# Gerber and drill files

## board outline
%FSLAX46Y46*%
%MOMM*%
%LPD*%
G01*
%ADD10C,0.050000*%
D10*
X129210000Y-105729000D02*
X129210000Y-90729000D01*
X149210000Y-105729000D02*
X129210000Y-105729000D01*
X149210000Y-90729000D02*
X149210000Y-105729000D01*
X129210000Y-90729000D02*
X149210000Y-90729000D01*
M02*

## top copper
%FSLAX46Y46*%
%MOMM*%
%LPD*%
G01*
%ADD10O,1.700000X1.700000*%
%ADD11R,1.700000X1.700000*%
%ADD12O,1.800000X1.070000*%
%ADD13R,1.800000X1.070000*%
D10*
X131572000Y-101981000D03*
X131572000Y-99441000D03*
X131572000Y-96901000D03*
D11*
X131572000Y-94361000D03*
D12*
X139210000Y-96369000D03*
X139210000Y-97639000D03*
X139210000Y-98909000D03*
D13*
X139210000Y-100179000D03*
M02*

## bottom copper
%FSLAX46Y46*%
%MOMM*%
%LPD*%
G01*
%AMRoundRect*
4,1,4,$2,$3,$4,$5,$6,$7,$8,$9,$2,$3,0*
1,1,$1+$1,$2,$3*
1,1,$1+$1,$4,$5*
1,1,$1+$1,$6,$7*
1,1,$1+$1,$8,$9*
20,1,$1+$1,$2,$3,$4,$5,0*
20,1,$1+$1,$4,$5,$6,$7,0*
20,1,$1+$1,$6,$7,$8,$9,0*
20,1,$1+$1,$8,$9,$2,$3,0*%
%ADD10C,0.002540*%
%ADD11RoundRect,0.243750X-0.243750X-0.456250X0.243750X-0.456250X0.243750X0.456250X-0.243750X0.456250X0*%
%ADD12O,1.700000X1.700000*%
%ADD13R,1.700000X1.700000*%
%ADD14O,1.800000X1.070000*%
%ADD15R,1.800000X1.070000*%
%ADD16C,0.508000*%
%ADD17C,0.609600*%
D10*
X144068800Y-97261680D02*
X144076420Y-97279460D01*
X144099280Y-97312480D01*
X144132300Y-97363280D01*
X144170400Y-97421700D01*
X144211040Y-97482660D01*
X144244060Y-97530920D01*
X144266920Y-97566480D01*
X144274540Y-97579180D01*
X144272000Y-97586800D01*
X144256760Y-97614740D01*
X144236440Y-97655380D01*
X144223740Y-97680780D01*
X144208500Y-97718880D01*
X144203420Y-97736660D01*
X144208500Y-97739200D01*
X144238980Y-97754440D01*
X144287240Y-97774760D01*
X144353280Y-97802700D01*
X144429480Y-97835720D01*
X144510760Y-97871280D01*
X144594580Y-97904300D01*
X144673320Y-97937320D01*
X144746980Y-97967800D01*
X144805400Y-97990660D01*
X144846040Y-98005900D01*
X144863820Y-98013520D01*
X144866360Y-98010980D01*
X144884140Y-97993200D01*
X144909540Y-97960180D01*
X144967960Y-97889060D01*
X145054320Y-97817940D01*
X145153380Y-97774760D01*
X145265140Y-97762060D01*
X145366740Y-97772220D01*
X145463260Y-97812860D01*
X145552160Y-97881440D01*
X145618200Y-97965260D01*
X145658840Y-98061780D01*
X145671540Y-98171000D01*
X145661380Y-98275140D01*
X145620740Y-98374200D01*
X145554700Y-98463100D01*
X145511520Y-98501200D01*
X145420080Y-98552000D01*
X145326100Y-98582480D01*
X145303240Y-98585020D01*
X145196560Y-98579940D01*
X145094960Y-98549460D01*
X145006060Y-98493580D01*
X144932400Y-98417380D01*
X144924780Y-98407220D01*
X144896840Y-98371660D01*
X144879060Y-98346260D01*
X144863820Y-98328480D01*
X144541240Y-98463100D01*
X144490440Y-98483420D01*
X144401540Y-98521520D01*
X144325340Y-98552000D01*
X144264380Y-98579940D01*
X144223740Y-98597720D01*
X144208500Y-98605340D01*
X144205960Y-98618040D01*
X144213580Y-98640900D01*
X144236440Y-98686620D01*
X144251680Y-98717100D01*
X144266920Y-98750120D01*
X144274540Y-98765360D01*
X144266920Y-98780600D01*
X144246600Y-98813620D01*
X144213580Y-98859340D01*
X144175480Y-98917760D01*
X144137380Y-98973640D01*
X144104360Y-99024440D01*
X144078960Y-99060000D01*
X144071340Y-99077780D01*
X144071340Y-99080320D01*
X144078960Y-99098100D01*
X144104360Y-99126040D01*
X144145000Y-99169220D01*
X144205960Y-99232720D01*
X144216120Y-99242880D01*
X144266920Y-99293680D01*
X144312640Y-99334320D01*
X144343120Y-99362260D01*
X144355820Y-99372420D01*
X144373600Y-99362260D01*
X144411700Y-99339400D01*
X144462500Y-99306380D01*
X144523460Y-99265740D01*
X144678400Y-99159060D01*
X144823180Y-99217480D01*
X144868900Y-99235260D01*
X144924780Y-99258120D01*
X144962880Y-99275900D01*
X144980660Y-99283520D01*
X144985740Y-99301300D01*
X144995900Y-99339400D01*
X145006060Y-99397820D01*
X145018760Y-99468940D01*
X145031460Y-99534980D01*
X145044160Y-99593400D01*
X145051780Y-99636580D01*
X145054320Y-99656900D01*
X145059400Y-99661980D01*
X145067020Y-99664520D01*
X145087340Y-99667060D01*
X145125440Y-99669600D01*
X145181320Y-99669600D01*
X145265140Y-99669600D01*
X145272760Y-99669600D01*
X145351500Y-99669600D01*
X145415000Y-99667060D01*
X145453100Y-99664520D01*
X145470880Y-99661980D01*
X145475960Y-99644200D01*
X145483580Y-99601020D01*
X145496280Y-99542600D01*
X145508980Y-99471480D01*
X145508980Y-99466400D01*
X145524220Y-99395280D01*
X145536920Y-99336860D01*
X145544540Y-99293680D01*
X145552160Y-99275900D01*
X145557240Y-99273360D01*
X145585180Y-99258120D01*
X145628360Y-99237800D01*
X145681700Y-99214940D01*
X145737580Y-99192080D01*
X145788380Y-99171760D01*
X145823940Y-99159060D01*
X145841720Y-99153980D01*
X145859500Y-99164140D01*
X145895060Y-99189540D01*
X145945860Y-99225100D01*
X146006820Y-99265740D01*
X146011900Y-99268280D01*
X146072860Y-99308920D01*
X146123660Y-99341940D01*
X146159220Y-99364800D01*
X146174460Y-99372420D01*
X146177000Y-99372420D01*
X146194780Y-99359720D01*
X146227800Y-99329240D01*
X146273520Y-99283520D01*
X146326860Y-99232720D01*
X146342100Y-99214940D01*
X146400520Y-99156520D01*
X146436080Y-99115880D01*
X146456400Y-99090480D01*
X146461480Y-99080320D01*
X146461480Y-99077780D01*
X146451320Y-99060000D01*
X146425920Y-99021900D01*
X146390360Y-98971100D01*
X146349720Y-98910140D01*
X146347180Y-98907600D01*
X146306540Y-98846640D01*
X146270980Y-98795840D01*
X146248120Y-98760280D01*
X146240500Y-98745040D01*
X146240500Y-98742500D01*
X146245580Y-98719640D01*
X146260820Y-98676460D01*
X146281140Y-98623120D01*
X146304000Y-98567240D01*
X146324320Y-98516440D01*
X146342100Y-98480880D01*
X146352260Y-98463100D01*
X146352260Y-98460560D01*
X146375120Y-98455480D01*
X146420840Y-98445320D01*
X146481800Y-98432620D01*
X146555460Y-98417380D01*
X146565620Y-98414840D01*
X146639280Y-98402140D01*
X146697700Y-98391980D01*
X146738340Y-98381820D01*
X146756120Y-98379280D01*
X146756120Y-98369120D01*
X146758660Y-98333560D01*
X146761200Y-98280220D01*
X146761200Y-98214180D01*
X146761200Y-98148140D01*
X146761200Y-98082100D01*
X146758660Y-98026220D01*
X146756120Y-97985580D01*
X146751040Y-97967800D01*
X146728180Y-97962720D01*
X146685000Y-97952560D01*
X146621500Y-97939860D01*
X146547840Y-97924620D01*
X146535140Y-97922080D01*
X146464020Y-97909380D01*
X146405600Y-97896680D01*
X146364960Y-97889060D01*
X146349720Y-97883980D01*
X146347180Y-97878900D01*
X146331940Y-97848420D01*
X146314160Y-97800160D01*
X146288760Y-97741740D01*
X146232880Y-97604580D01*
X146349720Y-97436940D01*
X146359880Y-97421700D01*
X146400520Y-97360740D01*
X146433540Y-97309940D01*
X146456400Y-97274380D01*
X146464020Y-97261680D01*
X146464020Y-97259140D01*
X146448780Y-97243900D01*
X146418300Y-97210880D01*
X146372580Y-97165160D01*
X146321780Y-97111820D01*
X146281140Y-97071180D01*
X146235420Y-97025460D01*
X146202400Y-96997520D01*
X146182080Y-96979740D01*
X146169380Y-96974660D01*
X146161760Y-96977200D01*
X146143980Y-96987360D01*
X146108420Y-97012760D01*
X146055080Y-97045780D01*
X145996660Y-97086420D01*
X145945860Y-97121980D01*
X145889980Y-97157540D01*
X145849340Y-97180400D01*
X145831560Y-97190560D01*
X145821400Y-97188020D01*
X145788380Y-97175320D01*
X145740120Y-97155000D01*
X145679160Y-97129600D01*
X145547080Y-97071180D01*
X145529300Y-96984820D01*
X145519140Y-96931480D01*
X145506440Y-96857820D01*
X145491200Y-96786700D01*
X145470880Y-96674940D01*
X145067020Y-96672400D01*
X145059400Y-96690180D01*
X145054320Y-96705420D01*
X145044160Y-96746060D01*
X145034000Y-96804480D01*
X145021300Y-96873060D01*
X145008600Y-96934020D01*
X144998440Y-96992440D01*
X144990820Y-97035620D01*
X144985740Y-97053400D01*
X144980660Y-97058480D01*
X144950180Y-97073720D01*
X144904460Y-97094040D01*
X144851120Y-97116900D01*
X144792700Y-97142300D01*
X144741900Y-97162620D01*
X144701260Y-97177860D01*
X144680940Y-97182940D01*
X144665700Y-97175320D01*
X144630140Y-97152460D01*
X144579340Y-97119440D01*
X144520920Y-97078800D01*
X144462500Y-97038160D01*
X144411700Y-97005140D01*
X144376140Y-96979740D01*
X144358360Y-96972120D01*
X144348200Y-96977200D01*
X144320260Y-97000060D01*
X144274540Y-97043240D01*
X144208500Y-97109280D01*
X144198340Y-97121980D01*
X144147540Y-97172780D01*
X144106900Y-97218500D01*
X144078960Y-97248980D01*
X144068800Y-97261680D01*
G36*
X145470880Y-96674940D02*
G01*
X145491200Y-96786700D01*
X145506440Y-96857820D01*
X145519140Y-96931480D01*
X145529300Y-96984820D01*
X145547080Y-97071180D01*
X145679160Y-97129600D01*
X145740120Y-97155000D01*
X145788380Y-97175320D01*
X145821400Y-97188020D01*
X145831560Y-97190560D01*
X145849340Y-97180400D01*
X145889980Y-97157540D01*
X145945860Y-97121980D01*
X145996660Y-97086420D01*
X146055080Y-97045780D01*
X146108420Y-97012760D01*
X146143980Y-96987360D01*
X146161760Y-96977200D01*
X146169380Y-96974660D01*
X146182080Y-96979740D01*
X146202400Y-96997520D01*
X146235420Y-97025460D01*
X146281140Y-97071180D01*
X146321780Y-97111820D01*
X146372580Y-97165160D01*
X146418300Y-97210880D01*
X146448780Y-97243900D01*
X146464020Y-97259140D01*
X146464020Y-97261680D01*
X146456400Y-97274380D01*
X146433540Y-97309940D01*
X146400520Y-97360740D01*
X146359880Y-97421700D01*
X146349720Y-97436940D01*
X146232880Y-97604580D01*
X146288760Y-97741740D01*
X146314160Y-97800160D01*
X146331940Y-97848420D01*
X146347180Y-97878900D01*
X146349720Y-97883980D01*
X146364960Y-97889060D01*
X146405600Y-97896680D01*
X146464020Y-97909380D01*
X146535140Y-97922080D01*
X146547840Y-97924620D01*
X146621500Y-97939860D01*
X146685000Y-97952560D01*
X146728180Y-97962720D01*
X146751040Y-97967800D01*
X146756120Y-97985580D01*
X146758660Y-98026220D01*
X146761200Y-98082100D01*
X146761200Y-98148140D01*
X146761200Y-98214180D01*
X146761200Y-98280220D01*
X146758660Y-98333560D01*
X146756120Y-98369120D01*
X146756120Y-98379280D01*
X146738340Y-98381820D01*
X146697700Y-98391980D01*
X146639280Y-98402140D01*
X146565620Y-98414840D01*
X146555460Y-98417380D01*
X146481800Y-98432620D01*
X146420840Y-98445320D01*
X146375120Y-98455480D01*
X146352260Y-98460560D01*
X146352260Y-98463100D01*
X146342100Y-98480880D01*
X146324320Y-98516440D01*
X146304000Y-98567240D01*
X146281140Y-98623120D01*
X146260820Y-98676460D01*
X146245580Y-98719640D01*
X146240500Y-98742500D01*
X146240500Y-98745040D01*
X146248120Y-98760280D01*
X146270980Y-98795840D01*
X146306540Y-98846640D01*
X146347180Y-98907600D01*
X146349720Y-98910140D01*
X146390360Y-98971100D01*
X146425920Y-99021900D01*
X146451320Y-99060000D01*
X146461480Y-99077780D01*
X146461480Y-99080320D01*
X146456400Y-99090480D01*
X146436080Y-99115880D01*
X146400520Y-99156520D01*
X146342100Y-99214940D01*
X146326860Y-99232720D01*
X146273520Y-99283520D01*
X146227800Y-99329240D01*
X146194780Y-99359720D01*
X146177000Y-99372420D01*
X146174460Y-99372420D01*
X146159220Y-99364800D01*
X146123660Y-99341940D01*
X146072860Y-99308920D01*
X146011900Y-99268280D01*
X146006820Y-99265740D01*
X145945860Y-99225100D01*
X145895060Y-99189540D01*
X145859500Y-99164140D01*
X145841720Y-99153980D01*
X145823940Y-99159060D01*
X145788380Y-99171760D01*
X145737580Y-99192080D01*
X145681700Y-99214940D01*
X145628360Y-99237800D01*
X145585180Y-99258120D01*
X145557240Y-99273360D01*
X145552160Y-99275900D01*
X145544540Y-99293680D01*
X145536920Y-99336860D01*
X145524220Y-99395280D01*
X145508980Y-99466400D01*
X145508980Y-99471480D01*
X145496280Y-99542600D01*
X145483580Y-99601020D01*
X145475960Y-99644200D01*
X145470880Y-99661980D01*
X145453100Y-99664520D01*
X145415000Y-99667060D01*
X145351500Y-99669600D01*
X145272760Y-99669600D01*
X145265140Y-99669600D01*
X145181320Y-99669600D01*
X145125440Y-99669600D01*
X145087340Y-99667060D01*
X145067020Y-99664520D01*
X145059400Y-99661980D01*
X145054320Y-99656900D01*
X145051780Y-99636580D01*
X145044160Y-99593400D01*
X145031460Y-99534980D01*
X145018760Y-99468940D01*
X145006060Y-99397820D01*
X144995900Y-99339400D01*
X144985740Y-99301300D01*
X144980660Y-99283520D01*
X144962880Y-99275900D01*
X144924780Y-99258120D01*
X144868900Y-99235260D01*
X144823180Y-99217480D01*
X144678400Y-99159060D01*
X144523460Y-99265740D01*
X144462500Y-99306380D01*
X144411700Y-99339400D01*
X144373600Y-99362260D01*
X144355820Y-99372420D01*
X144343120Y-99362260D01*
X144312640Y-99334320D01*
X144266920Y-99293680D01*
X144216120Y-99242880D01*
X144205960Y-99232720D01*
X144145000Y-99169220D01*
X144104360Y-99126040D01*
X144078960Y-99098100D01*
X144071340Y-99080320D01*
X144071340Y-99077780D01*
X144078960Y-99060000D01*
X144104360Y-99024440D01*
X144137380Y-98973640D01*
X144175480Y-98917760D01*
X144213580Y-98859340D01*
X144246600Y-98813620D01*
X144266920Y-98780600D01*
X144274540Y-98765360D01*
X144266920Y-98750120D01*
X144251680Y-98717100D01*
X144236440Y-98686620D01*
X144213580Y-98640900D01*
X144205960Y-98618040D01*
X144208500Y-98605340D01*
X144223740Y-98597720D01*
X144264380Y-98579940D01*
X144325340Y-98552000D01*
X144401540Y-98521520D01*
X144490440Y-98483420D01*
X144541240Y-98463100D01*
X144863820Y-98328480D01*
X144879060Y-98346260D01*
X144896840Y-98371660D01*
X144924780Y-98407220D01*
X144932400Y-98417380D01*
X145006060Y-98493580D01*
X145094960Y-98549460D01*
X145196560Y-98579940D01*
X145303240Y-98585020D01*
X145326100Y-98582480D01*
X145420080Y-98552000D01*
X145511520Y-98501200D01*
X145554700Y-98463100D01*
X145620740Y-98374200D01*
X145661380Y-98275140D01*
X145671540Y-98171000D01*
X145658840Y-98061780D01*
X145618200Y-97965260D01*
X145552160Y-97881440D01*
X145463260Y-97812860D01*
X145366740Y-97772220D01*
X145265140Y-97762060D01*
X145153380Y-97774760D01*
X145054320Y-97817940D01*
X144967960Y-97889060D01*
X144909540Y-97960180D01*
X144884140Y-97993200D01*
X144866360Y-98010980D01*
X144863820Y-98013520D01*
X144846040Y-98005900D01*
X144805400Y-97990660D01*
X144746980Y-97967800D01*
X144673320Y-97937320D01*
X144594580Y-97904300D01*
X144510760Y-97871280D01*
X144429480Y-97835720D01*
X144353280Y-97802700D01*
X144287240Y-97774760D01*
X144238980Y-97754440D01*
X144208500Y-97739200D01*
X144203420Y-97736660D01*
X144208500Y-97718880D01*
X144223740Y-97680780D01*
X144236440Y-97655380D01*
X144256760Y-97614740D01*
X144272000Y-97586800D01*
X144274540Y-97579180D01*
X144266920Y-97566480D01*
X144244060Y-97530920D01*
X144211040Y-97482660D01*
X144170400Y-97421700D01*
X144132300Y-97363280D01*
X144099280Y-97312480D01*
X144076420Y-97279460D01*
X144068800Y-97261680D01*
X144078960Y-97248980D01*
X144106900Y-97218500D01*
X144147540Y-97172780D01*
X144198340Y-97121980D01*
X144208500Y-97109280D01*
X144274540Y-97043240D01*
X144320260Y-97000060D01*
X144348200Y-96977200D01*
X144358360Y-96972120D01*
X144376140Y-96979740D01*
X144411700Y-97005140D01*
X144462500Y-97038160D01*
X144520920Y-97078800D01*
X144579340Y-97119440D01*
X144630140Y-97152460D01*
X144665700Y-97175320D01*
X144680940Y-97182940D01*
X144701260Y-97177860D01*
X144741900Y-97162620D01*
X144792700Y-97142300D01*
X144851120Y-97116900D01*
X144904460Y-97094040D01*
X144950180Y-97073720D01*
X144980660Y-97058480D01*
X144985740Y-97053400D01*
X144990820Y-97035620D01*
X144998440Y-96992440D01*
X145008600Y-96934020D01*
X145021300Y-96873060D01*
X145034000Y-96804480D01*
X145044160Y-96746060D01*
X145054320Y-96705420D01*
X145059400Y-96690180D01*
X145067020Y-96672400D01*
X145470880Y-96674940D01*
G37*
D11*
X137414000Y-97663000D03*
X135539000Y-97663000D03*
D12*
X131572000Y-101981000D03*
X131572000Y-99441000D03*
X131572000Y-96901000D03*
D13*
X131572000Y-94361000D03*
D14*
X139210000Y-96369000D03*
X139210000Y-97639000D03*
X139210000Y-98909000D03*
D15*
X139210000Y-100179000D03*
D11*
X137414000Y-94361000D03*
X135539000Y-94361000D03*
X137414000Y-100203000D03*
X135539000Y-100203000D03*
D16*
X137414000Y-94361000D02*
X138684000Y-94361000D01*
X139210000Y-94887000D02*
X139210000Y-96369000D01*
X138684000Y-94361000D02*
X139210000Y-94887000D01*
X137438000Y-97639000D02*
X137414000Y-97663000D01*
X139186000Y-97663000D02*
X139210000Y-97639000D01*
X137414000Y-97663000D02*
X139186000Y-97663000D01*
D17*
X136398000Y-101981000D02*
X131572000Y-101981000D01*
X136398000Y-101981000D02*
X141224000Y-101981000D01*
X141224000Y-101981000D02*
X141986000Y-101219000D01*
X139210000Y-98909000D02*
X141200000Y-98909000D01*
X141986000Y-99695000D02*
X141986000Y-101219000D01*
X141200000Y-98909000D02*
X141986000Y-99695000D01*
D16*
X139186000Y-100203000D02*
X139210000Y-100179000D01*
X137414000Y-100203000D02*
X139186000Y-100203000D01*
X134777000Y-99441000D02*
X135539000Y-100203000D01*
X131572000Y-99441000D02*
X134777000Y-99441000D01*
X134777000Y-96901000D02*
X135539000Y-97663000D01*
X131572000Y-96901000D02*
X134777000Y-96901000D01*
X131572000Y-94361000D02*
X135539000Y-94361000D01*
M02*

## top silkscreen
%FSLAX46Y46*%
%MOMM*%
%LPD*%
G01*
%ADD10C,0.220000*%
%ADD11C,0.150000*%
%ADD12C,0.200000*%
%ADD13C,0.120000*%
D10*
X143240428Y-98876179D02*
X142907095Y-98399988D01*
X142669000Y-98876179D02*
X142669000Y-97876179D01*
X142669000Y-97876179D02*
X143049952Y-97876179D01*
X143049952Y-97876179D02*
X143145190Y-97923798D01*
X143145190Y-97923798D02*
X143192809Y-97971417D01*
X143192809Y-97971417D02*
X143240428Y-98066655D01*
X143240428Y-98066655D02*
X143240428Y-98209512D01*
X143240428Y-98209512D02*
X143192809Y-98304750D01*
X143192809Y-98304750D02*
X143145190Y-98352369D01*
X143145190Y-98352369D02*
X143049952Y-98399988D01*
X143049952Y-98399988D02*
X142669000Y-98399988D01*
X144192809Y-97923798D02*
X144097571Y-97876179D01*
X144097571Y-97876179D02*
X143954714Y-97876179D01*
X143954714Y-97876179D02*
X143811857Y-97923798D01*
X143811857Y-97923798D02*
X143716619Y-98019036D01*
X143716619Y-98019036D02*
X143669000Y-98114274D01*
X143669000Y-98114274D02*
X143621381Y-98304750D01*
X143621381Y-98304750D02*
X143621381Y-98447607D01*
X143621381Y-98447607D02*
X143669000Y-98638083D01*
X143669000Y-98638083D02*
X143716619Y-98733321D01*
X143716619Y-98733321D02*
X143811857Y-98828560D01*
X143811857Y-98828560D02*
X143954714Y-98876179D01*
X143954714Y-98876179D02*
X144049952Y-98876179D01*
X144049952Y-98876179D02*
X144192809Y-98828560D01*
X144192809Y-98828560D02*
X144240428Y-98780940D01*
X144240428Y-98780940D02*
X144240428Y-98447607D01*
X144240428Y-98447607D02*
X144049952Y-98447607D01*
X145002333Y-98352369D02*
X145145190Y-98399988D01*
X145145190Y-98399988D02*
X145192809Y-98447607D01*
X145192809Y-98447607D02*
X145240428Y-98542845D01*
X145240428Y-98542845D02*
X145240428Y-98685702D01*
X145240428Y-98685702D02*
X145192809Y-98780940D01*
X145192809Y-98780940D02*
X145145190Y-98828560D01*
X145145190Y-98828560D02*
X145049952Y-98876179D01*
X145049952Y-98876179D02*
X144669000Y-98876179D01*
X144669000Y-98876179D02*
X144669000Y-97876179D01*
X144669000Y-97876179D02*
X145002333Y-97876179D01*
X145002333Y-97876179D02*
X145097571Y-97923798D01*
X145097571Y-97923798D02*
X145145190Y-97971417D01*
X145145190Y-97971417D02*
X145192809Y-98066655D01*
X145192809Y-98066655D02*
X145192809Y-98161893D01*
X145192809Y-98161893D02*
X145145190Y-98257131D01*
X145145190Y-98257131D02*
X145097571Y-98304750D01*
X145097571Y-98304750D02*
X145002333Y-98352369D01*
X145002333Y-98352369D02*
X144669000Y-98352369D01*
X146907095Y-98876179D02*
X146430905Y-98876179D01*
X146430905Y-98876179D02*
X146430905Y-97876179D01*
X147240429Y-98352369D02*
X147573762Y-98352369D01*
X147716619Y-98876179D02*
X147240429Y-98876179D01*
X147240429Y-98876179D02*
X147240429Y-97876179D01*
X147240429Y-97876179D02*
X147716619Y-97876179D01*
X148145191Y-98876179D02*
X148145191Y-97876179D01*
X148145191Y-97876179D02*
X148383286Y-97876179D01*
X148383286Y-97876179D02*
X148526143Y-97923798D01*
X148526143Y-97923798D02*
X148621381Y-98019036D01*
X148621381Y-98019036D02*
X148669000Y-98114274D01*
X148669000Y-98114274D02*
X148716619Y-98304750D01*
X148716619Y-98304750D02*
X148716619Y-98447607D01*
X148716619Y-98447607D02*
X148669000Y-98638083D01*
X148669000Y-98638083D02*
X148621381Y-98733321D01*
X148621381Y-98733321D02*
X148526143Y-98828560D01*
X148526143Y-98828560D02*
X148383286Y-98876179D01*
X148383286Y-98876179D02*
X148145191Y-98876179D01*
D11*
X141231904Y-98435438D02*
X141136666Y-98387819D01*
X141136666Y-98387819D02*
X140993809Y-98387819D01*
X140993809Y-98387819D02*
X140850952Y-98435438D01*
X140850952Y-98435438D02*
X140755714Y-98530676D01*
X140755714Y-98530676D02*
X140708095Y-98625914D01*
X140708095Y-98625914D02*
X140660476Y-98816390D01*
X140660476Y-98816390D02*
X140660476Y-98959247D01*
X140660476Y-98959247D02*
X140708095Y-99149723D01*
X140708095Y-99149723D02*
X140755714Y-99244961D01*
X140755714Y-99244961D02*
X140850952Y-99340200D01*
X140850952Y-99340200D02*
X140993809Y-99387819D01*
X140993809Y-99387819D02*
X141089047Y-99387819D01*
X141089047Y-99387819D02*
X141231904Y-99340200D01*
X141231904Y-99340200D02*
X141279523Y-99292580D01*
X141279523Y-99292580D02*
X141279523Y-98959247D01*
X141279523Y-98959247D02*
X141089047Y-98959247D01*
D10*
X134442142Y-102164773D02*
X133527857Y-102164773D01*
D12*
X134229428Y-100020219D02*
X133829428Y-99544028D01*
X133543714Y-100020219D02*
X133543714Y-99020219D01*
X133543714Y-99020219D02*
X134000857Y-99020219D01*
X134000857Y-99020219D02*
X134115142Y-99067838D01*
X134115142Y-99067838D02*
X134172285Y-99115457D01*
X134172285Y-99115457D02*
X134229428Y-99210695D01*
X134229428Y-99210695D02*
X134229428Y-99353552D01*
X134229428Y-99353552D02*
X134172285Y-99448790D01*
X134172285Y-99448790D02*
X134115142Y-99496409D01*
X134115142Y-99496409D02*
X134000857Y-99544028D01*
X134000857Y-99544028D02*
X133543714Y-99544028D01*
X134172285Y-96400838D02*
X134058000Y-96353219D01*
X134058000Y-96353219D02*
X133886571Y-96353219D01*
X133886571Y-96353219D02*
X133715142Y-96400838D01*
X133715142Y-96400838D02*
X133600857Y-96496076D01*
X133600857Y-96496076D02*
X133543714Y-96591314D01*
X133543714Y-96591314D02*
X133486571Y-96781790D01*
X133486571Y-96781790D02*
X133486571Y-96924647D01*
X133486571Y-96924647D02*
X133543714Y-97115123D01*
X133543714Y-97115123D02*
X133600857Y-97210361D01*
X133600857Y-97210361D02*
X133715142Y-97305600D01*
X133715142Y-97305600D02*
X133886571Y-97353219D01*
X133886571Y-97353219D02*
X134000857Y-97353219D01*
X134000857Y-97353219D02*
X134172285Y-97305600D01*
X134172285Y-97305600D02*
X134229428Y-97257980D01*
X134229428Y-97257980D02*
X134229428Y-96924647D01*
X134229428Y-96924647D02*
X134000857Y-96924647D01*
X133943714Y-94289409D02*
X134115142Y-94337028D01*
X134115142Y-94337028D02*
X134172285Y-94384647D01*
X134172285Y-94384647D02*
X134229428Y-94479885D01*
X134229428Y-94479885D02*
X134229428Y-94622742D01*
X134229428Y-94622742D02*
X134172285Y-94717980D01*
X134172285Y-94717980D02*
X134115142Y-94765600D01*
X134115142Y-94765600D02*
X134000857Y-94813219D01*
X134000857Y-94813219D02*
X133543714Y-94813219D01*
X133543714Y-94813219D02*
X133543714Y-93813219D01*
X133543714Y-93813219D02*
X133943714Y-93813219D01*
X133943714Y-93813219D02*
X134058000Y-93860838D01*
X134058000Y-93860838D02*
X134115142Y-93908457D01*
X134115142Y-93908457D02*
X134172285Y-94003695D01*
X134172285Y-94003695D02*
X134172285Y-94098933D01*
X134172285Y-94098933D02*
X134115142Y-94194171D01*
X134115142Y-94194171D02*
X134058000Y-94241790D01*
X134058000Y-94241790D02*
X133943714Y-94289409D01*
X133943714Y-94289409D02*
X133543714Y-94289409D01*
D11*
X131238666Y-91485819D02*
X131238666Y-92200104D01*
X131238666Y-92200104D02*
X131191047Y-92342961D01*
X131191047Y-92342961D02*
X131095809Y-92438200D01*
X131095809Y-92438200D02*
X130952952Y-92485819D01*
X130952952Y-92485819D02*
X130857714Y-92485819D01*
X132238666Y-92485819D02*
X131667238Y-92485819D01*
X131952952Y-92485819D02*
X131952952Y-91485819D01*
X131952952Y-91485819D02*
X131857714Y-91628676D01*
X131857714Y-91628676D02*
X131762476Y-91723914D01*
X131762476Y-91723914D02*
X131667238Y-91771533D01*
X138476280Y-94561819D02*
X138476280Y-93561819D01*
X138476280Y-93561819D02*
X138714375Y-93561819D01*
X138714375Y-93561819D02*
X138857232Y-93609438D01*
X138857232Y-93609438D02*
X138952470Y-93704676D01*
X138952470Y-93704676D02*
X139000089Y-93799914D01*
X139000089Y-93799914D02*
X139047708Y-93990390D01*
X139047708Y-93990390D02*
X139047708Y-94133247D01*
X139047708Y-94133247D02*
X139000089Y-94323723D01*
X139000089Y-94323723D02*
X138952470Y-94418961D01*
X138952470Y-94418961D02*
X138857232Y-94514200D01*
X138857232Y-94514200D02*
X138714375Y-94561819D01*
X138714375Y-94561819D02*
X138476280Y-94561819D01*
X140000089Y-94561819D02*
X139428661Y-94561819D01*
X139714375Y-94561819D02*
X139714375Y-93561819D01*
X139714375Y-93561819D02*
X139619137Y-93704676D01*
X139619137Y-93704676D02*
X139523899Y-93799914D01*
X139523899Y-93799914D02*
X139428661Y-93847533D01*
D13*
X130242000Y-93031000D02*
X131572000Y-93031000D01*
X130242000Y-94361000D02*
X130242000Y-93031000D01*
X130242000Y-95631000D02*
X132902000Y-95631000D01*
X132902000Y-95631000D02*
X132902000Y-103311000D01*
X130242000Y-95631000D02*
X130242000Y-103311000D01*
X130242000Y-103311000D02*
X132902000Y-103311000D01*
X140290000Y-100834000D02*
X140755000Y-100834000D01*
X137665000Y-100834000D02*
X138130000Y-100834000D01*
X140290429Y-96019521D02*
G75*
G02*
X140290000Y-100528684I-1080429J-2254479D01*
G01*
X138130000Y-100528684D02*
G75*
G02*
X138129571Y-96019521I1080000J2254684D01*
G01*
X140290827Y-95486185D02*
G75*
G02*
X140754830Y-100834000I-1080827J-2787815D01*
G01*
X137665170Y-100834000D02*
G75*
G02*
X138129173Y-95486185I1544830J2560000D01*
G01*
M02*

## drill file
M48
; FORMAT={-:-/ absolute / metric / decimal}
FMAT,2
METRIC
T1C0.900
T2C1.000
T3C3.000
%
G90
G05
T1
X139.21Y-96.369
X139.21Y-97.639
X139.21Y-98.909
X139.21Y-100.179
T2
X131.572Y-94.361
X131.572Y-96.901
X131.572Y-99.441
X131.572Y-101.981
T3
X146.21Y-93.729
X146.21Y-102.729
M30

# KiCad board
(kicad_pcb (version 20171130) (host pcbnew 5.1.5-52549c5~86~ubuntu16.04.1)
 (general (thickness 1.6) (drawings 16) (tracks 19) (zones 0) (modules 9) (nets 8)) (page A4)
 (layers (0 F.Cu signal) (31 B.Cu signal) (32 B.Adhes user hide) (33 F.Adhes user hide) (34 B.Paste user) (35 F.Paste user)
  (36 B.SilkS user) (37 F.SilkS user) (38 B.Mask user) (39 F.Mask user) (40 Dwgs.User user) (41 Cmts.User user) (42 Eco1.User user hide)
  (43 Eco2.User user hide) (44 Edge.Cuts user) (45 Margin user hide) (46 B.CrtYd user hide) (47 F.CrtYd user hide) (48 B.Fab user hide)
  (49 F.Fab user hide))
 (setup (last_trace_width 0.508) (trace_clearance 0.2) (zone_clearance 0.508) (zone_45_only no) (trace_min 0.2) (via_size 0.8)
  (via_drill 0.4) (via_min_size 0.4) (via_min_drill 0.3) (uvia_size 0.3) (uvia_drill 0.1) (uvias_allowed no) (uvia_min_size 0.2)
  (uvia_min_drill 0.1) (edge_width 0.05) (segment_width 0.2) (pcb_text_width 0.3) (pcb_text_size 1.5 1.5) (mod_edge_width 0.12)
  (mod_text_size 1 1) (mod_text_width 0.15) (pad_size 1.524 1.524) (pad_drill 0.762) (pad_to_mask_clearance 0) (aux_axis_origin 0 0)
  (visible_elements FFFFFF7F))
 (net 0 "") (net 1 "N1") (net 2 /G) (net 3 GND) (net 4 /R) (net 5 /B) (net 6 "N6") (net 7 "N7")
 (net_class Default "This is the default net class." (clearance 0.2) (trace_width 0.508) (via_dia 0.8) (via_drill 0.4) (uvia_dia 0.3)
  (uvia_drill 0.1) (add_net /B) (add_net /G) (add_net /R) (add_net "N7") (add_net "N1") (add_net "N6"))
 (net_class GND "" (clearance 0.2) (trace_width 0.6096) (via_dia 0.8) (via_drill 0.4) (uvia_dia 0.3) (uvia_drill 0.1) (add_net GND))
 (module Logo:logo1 (layer B.Cu) (at 141.986 98.171 90)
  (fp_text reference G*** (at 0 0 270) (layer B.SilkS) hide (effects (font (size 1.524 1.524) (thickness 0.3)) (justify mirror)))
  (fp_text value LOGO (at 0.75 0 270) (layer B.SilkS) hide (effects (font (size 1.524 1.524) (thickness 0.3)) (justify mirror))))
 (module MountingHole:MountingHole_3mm (layer F.Cu) (at 146.21 102.729)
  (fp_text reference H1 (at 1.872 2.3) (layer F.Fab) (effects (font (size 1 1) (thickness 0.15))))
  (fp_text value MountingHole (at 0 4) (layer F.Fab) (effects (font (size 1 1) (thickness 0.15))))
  (pad 1 np_thru_hole circle (at 0 0) (size 3 3) (drill 3) (layers *.Cu *.Mask)))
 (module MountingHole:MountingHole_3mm (layer F.Cu) (at 146.21 93.729)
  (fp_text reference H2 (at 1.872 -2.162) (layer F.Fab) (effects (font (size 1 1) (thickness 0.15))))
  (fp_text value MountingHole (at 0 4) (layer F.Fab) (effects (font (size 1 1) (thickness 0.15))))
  (pad 1 np_thru_hole circle (at 0 0) (size 3 3) (drill 3) (layers *.Cu *.Mask)))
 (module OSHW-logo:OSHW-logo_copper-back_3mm (layer B.Cu) (at 145.415 98.171 90)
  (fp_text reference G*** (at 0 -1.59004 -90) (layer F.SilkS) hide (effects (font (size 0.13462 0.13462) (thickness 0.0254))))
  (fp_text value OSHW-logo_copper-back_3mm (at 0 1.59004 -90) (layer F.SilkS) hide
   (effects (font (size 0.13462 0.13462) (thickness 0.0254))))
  (fp_poly
   (pts (xy 0.90932 -1.3462) (xy 0.89154 -1.33858) (xy 0.85852 -1.31572) (xy 0.80772 -1.2827) (xy 0.7493 -1.2446) (xy 0.68834 -1.20396)
    (xy 0.64008 -1.17094) (xy 0.60452 -1.14808) (xy 0.59182 -1.14046) (xy 0.5842 -1.143) (xy 0.55626 -1.15824) (xy 0.51562 -1.17856)
    (xy 0.49022 -1.19126) (xy 0.45212 -1.2065) (xy 0.43434 -1.21158) (xy 0.4318 -1.2065) (xy 0.41656 -1.17602) (xy 0.39624 -1.12776)
    (xy 0.3683 -1.06172) (xy 0.33528 -0.98552) (xy 0.29972 -0.90424) (xy 0.2667 -0.82042) (xy 0.23368 -0.74168) (xy 0.2032 -0.66802)
    (xy 0.18034 -0.6096) (xy 0.1651 -0.56896) (xy 0.15748 -0.55118) (xy 0.16002 -0.54864) (xy 0.1778 -0.53086) (xy 0.21082 -0.50546)
    (xy 0.28194 -0.44704) (xy 0.35306 -0.36068) (xy 0.39624 -0.26162) (xy 0.40894 -0.14986) (xy 0.39878 -0.04826) (xy 0.35814 0.04826)
    (xy 0.28956 0.13716) (xy 0.20574 0.2032) (xy 0.10922 0.24384) (xy 0 0.25654) (xy -0.10414 0.24638) (xy -0.2032 0.20574)
    (xy -0.2921 0.1397) (xy -0.3302 0.09652) (xy -0.381 0.00508) (xy -0.41148 -0.0889) (xy -0.41402 -0.11176) (xy -0.40894 -0.21844)
    (xy -0.37846 -0.32004) (xy -0.32258 -0.40894) (xy -0.24638 -0.4826) (xy -0.23622 -0.49022) (xy -0.20066 -0.51816) (xy -0.17526 -0.53594)
    (xy -0.15748 -0.55118) (xy -0.2921 -0.87376) (xy -0.31242 -0.92456) (xy -0.35052 -1.01346) (xy -0.381 -1.08966) (xy -0.40894 -1.15062)
    (xy -0.42672 -1.19126) (xy -0.43434 -1.2065) (xy -0.44704 -1.20904) (xy -0.4699 -1.20142) (xy -0.51562 -1.17856) (xy -0.5461 -1.16332)
    (xy -0.57912 -1.14808) (xy -0.59436 -1.14046) (xy -0.6096 -1.14808) (xy -0.64262 -1.1684) (xy -0.68834 -1.20142) (xy -0.74676 -1.23952)
    (xy -0.80264 -1.27762) (xy -0.85344 -1.31064) (xy -0.889 -1.33604) (xy -0.90678 -1.34366) (xy -0.90932 -1.34366) (xy -0.9271 -1.33604)
    (xy -0.95504 -1.31064) (xy -0.99822 -1.27) (xy -1.06172 -1.20904) (xy -1.07188 -1.19888) (xy -1.12268 -1.14808) (xy -1.16332 -1.10236)
    (xy -1.19126 -1.07188) (xy -1.20142 -1.05918) (xy -1.19126 -1.0414) (xy -1.1684 -1.0033) (xy -1.13538 -0.9525) (xy -1.09474 -0.89154)
    (xy -0.98806 -0.7366) (xy -1.04648 -0.59182) (xy -1.06426 -0.5461) (xy -1.08712 -0.49022) (xy -1.1049 -0.45212) (xy -1.11252 -0.43434)
    (xy -1.1303 -0.42926) (xy -1.1684 -0.4191) (xy -1.22682 -0.40894) (xy -1.29794 -0.39624) (xy -1.36398 -0.38354) (xy -1.4224 -0.37084)
    (xy -1.46558 -0.36322) (xy -1.4859 -0.36068) (xy -1.49098 -0.3556) (xy -1.49352 -0.34798) (xy -1.49606 -0.32766) (xy -1.4986 -0.28956)
    (xy -1.4986 -0.23368) (xy -1.4986 -0.14986) (xy -1.4986 -0.14224) (xy -1.4986 -0.0635) (xy -1.49606 0) (xy -1.49352 0.0381)
    (xy -1.49098 0.05588) (xy -1.4732 0.06096) (xy -1.43002 0.06858) (xy -1.3716 0.08128) (xy -1.30048 0.09398) (xy -1.2954 0.09398)
    (xy -1.22428 0.10922) (xy -1.16586 0.12192) (xy -1.12268 0.12954) (xy -1.1049 0.13716) (xy -1.10236 0.14224) (xy -1.08712 0.17018)
    (xy -1.0668 0.21336) (xy -1.04394 0.2667) (xy -1.02108 0.32258) (xy -1.00076 0.37338) (xy -0.98806 0.40894) (xy -0.98298 0.42672)
    (xy -0.99314 0.4445) (xy -1.01854 0.48006) (xy -1.0541 0.53086) (xy -1.09474 0.59182) (xy -1.09728 0.5969) (xy -1.13792 0.65786)
    (xy -1.17094 0.70866) (xy -1.1938 0.74422) (xy -1.20142 0.75946) (xy -1.20142 0.762) (xy -1.18872 0.77978) (xy -1.15824 0.8128)
    (xy -1.11252 0.85852) (xy -1.06172 0.91186) (xy -1.04394 0.9271) (xy -0.98552 0.98552) (xy -0.94488 1.02108) (xy -0.91948 1.0414)
    (xy -0.90932 1.04648) (xy -0.90678 1.04648) (xy -0.889 1.03632) (xy -0.8509 1.01092) (xy -0.8001 0.97536) (xy -0.73914 0.93472)
    (xy -0.7366 0.93218) (xy -0.67564 0.89154) (xy -0.62484 0.85598) (xy -0.58928 0.83312) (xy -0.57404 0.8255) (xy -0.5715 0.8255)
    (xy -0.54864 0.83058) (xy -0.50546 0.84582) (xy -0.45212 0.86614) (xy -0.39624 0.889) (xy -0.34544 0.90932) (xy -0.30988 0.9271)
    (xy -0.2921 0.93726) (xy -0.28956 0.93726) (xy -0.28448 0.96012) (xy -0.27432 1.00584) (xy -0.26162 1.0668) (xy -0.24638 1.14046)
    (xy -0.24384 1.15062) (xy -0.23114 1.22428) (xy -0.22098 1.2827) (xy -0.21082 1.32334) (xy -0.20828 1.34112) (xy -0.19812 1.34112)
    (xy -0.16256 1.34366) (xy -0.10922 1.3462) (xy -0.04318 1.3462) (xy 0.02286 1.3462) (xy 0.0889 1.3462) (xy 0.14478 1.34366)
    (xy 0.18542 1.34112) (xy 0.2032 1.33604) (xy 0.20828 1.31318) (xy 0.21844 1.27) (xy 0.23114 1.2065) (xy 0.24638 1.13284)
    (xy 0.24892 1.12014) (xy 0.26162 1.04902) (xy 0.27432 0.9906) (xy 0.28194 0.94996) (xy 0.28702 0.93472) (xy 0.2921 0.93218)
    (xy 0.32258 0.91694) (xy 0.37084 0.89916) (xy 0.42926 0.87376) (xy 0.56642 0.81788) (xy 0.73406 0.93472) (xy 0.7493 0.94488)
    (xy 0.81026 0.98552) (xy 0.86106 1.01854) (xy 0.89662 1.0414) (xy 0.90932 1.04902) (xy 0.91186 1.04902) (xy 0.9271 1.03378)
    (xy 0.96012 1.0033) (xy 1.00584 0.95758) (xy 1.05918 0.90678) (xy 1.09982 0.86614) (xy 1.14554 0.82042) (xy 1.17348 0.7874)
    (xy 1.19126 0.76708) (xy 1.19634 0.75438) (xy 1.1938 0.74676) (xy 1.18364 0.72898) (xy 1.15824 0.69342) (xy 1.12522 0.64008)
    (xy 1.08458 0.58166) (xy 1.04902 0.53086) (xy 1.01346 0.47498) (xy 0.9906 0.43434) (xy 0.98044 0.41656) (xy 0.98298 0.4064)
    (xy 0.99568 0.37338) (xy 1.016 0.32512) (xy 1.0414 0.26416) (xy 1.09982 0.13208) (xy 1.18618 0.1143) (xy 1.23952 0.10414)
    (xy 1.31318 0.09144) (xy 1.3843 0.0762) (xy 1.49606 0.05588) (xy 1.4986 -0.34798) (xy 1.48082 -0.3556) (xy 1.46558 -0.36068)
    (xy 1.42494 -0.37084) (xy 1.36652 -0.381) (xy 1.29794 -0.3937) (xy 1.23698 -0.4064) (xy 1.17856 -0.41656) (xy 1.13538 -0.42418)
    (xy 1.1176 -0.42926) (xy 1.11252 -0.43434) (xy 1.09728 -0.46482) (xy 1.07696 -0.51054) (xy 1.0541 -0.56388) (xy 1.0287 -0.6223)
    (xy 1.00838 -0.6731) (xy 0.99314 -0.71374) (xy 0.98806 -0.73406) (xy 0.99568 -0.7493) (xy 1.01854 -0.78486) (xy 1.05156 -0.83566)
    (xy 1.0922 -0.89408) (xy 1.13284 -0.9525) (xy 1.16586 -1.0033) (xy 1.19126 -1.03886) (xy 1.19888 -1.05664) (xy 1.1938 -1.0668)
    (xy 1.17094 -1.09474) (xy 1.12776 -1.14046) (xy 1.06172 -1.2065) (xy 1.04902 -1.21666) (xy 0.99822 -1.26746) (xy 0.9525 -1.3081)
    (xy 0.92202 -1.33604) (xy 0.90932 -1.3462))
   (layer B.Cu) (width 0.00254)))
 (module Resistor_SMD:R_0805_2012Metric (layer B.Cu) (at 136.4765 97.663)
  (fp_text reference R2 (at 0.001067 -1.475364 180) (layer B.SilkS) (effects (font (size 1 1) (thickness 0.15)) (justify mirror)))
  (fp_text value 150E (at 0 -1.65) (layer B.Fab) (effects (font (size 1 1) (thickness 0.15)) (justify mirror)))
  (pad 2 smd roundrect (at 0.9375 0) (size 0.975 1.4) (layers B.Cu B.Paste B.Mask) (roundrect_rratio 0.25) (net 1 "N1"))
  (pad 1 smd roundrect (at -0.9375 0) (size 0.975 1.4) (layers B.Cu B.Paste B.Mask) (roundrect_rratio 0.25) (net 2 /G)))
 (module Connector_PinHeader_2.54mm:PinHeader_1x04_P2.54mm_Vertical (layer F.Cu) (at 131.572 94.361)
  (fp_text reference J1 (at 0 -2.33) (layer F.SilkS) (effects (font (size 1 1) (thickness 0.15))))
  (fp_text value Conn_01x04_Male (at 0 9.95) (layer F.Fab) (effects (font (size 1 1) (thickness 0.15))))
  (fp_line (start -1.33 -1.33) (end 0 -1.33) (layer F.SilkS) (width 0.12))
  (fp_line (start -1.33 0) (end -1.33 -1.33) (layer F.SilkS) (width 0.12))
  (fp_line (start -1.33 1.27) (end 1.33 1.27) (layer F.SilkS) (width 0.12))
  (fp_line (start 1.33 1.27) (end 1.33 8.95) (layer F.SilkS) (width 0.12))
  (fp_line (start -1.33 1.27) (end -1.33 8.95) (layer F.SilkS) (width 0.12))
  (fp_line (start -1.33 8.95) (end 1.33 8.95) (layer F.SilkS) (width 0.12))
  (pad 4 thru_hole oval (at 0 7.62) (size 1.7 1.7) (drill 1) (layers *.Cu *.Mask) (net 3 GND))
  (pad 3 thru_hole oval (at 0 5.08) (size 1.7 1.7) (drill 1) (layers *.Cu *.Mask) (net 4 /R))
  (pad 2 thru_hole oval (at 0 2.54) (size 1.7 1.7) (drill 1) (layers *.Cu *.Mask) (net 2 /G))
  (pad 1 thru_hole rect (at 0 0) (size 1.7 1.7) (drill 1) (layers *.Cu *.Mask) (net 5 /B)))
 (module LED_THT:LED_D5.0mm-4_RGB (layer F.Cu) (at 139.21 100.179 90)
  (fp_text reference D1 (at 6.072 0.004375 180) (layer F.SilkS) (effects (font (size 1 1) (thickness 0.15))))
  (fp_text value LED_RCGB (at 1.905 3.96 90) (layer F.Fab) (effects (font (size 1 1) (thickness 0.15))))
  (fp_line (start -0.655 1.08) (end -0.655 1.545) (layer F.SilkS) (width 0.12))
  (fp_line (start -0.655 -1.545) (end -0.655 -1.08) (layer F.SilkS) (width 0.12))
  (fp_arc (start 1.905 0) (end -0.349684 1.08) (angle -128.8) (layer F.SilkS) (width 0.12))
  (fp_arc (start 1.905 0) (end -0.349684 -1.08) (angle 128.8) (layer F.SilkS) (width 0.12))
  (fp_arc (start 1.905 0) (end -0.655 1.54483) (angle -127.7) (layer F.SilkS) (width 0.12))
  (fp_arc (start 1.905 0) (end -0.655 -1.54483) (angle 127.7) (layer F.SilkS) (width 0.12))
  (pad 4 thru_hole oval (at 3.81 0 90) (size 1.07 1.8) (drill 0.9) (layers *.Cu *.Mask) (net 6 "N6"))
  (pad 3 thru_hole oval (at 2.54 0 90) (size 1.07 1.8) (drill 0.9) (layers *.Cu *.Mask) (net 1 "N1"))
  (pad 2 thru_hole oval (at 1.27 0 90) (size 1.07 1.8) (drill 0.9) (layers *.Cu *.Mask) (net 3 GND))
  (pad 1 thru_hole rect (at 0 0 90) (size 1.07 1.8) (drill 0.9) (layers *.Cu *.Mask) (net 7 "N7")))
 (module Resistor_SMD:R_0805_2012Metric (layer B.Cu) (at 136.4765 94.361)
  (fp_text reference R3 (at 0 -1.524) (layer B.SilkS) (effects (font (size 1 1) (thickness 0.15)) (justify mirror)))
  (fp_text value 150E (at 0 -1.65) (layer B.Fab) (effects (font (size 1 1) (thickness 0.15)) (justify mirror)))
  (pad 2 smd roundrect (at 0.9375 0) (size 0.975 1.4) (layers B.Cu B.Paste B.Mask) (roundrect_rratio 0.25) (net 6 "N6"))
  (pad 1 smd roundrect (at -0.9375 0) (size 0.975 1.4) (layers B.Cu B.Paste B.Mask) (roundrect_rratio 0.25) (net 5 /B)))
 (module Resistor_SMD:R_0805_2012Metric (layer B.Cu) (at 136.4765 100.203)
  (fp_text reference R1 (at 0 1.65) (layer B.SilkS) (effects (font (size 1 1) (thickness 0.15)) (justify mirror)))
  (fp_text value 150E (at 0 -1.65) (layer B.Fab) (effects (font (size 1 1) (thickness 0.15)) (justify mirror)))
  (pad 2 smd roundrect (at 0.9375 0) (size 0.975 1.4) (layers B.Cu B.Paste B.Mask) (roundrect_rratio 0.25) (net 7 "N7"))
  (pad 1 smd roundrect (at -0.9375 0) (size 0.975 1.4) (layers B.Cu B.Paste B.Mask) (roundrect_rratio 0.25) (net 4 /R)))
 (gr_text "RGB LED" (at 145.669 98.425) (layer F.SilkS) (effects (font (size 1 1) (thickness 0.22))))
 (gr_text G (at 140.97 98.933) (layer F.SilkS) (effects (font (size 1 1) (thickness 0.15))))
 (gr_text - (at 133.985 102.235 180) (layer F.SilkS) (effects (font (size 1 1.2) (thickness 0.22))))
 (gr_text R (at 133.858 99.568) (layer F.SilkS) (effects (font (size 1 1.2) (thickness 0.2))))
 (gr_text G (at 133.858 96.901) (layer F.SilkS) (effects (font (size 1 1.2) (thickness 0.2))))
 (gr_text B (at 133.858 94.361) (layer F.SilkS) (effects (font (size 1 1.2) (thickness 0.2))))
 (gr_line (start 129.21 105.729) (end 129.21 90.729) (layer Edge.Cuts) (width 0.05))
 (gr_line (start 149.21 105.729) (end 129.21 105.729) (layer Edge.Cuts) (width 0.05))
 (gr_line (start 149.21 90.729) (end 149.21 105.729) (layer Edge.Cuts) (width 0.05))
 (gr_line (start 129.21 90.729) (end 149.21 90.729) (layer Edge.Cuts) (width 0.05))
 (segment (start 137.414 94.361) (end 138.684 94.361) (width 0.508) (layer B.Cu) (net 6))
 (segment (start 139.21 94.887) (end 139.21 96.369) (width 0.508) (layer B.Cu) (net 6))
 (segment (start 138.684 94.361) (end 139.21 94.887) (width 0.508) (layer B.Cu) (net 6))
 (segment (start 137.438 97.639) (end 137.414 97.663) (width 0.508) (layer B.Cu) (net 1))
 (segment (start 139.186 97.663) (end 139.21 97.639) (width 0.508) (layer B.Cu) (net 1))
 (segment (start 137.414 97.663) (end 139.186 97.663) (width 0.508) (layer B.Cu) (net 1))
 (segment (start 136.398 101.981) (end 131.572 101.981) (width 0.6096) (layer B.Cu) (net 3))
 (segment (start 136.398 101.981) (end 141.224 101.981) (width 0.6096) (layer B.Cu) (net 3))
 (segment (start 141.224 101.981) (end 141.986 101.219) (width 0.6096) (layer B.Cu) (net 3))
 (segment (start 139.21 98.909) (end 141.2 98.909) (width 0.6096) (layer B.Cu) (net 3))
 (segment (start 141.986 99.695) (end 141.986 101.219) (width 0.6096) (layer B.Cu) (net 3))
 (segment (start 141.2 98.909) (end 141.986 99.695) (width 0.6096) (layer B.Cu) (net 3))
 (segment (start 139.186 100.203) (end 139.21 100.179) (width 0.508) (layer B.Cu) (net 7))
 (segment (start 137.414 100.203) (end 139.186 100.203) (width 0.508) (layer B.Cu) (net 7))
 (segment (start 134.777 99.441) (end 135.539 100.203) (width 0.508) (layer B.Cu) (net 4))
 (segment (start 131.572 99.441) (end 134.777 99.441) (width 0.508) (layer B.Cu) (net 4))
 (segment (start 134.777 96.901) (end 135.539 97.663) (width 0.508) (layer B.Cu) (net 2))
 (segment (start 131.572 96.901) (end 134.777 96.901) (width 0.508) (layer B.Cu) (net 2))
 (segment (start 131.572 94.361) (end 135.539 94.361) (width 0.508) (layer B.Cu) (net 5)))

